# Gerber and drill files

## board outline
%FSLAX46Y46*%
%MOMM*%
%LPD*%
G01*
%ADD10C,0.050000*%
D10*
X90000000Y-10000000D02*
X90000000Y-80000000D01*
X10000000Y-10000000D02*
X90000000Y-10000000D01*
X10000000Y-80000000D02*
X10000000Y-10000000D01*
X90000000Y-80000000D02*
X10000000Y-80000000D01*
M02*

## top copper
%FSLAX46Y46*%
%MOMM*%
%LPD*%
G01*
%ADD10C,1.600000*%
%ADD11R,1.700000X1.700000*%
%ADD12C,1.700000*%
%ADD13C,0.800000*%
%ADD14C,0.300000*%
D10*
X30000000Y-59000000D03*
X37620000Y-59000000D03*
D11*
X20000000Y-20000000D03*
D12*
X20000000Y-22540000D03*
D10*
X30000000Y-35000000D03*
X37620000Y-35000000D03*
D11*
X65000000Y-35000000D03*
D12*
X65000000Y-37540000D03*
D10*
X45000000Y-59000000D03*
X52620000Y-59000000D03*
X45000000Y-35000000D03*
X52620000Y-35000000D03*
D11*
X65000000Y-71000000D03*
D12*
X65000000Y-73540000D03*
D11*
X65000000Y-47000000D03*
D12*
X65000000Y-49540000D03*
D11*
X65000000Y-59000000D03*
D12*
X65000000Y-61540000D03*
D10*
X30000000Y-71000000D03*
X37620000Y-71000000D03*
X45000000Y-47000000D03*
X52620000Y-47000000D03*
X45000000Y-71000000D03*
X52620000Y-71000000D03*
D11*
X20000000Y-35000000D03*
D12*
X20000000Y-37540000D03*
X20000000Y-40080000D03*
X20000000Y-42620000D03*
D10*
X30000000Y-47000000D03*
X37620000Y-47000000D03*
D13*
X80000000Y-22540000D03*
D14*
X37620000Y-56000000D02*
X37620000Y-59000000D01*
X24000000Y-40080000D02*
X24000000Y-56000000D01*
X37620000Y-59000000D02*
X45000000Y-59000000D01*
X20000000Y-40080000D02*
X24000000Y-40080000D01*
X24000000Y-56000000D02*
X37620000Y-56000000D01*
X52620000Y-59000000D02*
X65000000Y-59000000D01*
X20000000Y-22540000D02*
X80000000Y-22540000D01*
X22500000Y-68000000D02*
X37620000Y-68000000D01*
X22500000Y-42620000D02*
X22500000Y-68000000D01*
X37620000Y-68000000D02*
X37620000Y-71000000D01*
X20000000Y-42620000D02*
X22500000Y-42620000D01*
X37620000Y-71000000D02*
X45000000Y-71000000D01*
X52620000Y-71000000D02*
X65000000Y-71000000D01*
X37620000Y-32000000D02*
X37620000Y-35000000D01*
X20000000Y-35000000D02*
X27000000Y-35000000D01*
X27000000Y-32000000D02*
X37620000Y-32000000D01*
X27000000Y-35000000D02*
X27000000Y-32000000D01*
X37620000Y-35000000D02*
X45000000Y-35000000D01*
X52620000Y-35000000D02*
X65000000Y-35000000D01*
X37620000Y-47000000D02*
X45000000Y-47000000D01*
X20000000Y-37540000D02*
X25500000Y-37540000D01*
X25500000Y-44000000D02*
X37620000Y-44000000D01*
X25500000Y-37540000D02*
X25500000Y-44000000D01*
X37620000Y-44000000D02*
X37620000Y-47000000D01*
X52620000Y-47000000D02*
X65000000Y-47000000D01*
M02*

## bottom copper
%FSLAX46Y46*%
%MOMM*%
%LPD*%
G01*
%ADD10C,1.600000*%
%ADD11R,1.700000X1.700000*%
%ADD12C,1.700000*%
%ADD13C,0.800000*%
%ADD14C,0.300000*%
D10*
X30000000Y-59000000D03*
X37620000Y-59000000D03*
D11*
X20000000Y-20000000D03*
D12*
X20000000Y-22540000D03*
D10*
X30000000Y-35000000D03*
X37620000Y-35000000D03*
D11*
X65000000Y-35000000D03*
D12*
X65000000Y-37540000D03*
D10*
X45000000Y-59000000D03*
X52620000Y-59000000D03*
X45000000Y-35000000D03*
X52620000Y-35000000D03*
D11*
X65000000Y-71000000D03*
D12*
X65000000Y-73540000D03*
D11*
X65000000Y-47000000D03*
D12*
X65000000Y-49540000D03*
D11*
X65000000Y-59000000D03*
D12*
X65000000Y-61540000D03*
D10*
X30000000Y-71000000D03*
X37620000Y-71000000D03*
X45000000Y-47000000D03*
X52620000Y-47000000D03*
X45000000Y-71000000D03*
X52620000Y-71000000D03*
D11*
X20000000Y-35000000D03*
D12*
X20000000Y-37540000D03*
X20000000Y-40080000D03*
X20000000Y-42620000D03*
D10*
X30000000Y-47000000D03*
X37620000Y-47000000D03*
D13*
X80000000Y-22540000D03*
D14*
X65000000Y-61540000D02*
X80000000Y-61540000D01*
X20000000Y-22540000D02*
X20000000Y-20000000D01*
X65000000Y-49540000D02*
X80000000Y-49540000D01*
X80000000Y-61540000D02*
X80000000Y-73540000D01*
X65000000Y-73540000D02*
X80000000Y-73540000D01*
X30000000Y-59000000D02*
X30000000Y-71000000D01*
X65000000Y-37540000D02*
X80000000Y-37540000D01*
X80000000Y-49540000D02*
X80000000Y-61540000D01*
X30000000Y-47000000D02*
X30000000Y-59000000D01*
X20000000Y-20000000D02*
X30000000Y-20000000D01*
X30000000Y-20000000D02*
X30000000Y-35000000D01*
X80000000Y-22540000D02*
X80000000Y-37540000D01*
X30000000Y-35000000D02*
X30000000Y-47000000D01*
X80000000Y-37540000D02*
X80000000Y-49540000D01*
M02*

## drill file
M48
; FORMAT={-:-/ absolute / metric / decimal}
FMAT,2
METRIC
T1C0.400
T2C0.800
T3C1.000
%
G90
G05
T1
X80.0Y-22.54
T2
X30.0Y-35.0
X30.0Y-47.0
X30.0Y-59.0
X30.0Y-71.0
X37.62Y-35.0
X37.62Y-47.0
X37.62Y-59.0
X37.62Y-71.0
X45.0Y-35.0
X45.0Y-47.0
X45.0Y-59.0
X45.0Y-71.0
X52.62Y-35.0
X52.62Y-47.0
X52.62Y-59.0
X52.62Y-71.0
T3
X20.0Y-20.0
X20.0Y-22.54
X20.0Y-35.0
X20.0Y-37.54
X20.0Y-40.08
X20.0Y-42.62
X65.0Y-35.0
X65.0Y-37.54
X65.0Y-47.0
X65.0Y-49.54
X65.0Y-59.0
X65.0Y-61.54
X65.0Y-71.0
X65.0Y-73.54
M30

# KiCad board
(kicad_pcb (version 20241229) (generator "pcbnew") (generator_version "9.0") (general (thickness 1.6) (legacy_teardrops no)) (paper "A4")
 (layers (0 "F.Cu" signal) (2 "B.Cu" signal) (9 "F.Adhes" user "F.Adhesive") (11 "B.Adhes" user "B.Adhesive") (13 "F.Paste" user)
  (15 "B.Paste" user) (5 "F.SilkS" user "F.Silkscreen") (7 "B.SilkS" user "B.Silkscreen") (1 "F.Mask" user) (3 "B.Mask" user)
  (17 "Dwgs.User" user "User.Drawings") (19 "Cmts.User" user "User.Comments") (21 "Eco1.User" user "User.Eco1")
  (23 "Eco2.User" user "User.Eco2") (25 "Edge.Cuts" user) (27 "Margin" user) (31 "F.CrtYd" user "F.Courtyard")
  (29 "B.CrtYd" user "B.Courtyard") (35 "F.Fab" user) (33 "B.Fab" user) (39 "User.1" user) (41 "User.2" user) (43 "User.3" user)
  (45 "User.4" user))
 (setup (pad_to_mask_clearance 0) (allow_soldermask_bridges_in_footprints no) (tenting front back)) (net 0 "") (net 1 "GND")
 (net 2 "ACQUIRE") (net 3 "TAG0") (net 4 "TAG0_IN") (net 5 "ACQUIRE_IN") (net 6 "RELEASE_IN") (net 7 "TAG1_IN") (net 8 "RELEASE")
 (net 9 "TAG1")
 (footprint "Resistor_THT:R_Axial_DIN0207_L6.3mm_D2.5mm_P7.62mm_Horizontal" (layer "F.Cu") (at 30 59)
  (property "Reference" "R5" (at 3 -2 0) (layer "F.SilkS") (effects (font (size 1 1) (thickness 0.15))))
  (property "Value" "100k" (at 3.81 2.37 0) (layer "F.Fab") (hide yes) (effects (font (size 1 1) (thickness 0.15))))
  (pad "1" thru_hole circle (at 0 0) (size 1.6 1.6) (drill 0.8) (layers "*.Cu" "*.Mask") (remove_unused_layers no) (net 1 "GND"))
  (pad "2" thru_hole circle (at 7.62 0) (size 1.6 1.6) (drill 0.8) (layers "*.Cu" "*.Mask") (remove_unused_layers no) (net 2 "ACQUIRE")))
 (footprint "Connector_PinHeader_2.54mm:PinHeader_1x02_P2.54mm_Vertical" (layer "F.Cu") (at 20 20)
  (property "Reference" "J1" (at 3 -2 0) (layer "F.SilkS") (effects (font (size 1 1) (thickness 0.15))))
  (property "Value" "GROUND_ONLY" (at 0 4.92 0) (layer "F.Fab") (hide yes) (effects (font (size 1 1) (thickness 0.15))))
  (pad "1" thru_hole rect (at 0 0) (size 1.7 1.7) (drill 1) (layers "*.Cu" "*.Mask") (remove_unused_layers no) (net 1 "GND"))
  (pad "2" thru_hole circle (at 0 2.54) (size 1.7 1.7) (drill 1) (layers "*.Cu" "*.Mask") (remove_unused_layers no) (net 1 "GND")))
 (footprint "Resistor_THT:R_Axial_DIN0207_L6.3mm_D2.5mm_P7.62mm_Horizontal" (layer "F.Cu") (at 30 35)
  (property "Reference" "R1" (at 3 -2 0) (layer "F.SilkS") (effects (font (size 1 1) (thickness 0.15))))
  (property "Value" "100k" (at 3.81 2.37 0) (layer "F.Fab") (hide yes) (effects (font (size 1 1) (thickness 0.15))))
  (pad "1" thru_hole circle (at 0 0) (size 1.6 1.6) (drill 0.8) (layers "*.Cu" "*.Mask") (remove_unused_layers no) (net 1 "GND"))
  (pad "2" thru_hole circle (at 7.62 0) (size 1.6 1.6) (drill 0.8) (layers "*.Cu" "*.Mask") (remove_unused_layers no) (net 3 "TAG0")))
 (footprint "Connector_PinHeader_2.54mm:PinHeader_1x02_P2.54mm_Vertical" (layer "F.Cu") (at 65 35)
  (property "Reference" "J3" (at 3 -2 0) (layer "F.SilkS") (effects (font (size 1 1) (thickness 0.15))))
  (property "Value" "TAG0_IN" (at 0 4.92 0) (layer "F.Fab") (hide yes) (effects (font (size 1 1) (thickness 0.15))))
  (pad "1" thru_hole rect (at 0 0) (size 1.7 1.7) (drill 1) (layers "*.Cu" "*.Mask") (remove_unused_layers no) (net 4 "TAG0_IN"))
  (pad "2" thru_hole circle (at 0 2.54) (size 1.7 1.7) (drill 1) (layers "*.Cu" "*.Mask") (remove_unused_layers no) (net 1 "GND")))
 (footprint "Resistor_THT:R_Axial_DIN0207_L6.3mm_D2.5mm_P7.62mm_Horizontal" (layer "F.Cu") (at 45 59)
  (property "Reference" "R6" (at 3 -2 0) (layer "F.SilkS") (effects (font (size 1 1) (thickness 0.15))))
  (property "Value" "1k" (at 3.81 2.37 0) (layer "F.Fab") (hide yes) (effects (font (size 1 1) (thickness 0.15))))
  (pad "1" thru_hole circle (at 0 0) (size 1.6 1.6) (drill 0.8) (layers "*.Cu" "*.Mask") (remove_unused_layers no) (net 2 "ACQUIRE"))
  (pad "2" thru_hole circle (at 7.62 0) (size 1.6 1.6) (drill 0.8) (layers "*.Cu" "*.Mask") (remove_unused_layers no) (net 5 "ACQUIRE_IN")))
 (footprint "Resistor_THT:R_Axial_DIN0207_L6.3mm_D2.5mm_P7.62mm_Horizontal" (layer "F.Cu") (at 45 35)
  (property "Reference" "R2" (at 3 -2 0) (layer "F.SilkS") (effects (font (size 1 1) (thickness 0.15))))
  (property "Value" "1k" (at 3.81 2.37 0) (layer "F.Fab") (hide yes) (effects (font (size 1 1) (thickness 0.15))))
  (pad "1" thru_hole circle (at 0 0) (size 1.6 1.6) (drill 0.8) (layers "*.Cu" "*.Mask") (remove_unused_layers no) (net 3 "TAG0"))
  (pad "2" thru_hole circle (at 7.62 0) (size 1.6 1.6) (drill 0.8) (layers "*.Cu" "*.Mask") (remove_unused_layers no) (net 4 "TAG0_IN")))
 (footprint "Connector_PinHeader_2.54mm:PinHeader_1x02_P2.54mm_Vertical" (layer "F.Cu") (at 65 71)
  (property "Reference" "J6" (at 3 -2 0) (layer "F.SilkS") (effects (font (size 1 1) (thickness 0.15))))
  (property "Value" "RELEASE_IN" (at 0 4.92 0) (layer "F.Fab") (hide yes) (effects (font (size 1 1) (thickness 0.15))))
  (pad "1" thru_hole rect (at 0 0) (size 1.7 1.7) (drill 1) (layers "*.Cu" "*.Mask") (remove_unused_layers no) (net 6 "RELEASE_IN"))
  (pad "2" thru_hole circle (at 0 2.54) (size 1.7 1.7) (drill 1) (layers "*.Cu" "*.Mask") (remove_unused_layers no) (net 1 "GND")))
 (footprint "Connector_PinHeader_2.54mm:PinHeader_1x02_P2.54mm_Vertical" (layer "F.Cu") (at 65 47)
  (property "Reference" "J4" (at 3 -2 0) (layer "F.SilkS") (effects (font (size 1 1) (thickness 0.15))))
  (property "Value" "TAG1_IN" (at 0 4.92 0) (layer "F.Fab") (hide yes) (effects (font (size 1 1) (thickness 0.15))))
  (pad "1" thru_hole rect (at 0 0) (size 1.7 1.7) (drill 1) (layers "*.Cu" "*.Mask") (remove_unused_layers no) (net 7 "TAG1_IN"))
  (pad "2" thru_hole circle (at 0 2.54) (size 1.7 1.7) (drill 1) (layers "*.Cu" "*.Mask") (remove_unused_layers no) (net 1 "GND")))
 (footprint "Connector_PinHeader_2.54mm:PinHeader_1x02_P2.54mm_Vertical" (layer "F.Cu") (at 65 59)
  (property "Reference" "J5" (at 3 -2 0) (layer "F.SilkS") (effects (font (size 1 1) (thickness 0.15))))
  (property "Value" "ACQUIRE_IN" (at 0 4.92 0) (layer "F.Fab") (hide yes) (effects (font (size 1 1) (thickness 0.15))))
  (pad "1" thru_hole rect (at 0 0) (size 1.7 1.7) (drill 1) (layers "*.Cu" "*.Mask") (remove_unused_layers no) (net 5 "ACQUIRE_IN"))
  (pad "2" thru_hole circle (at 0 2.54) (size 1.7 1.7) (drill 1) (layers "*.Cu" "*.Mask") (remove_unused_layers no) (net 1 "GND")))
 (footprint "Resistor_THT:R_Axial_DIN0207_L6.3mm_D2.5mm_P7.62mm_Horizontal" (layer "F.Cu") (at 30 71)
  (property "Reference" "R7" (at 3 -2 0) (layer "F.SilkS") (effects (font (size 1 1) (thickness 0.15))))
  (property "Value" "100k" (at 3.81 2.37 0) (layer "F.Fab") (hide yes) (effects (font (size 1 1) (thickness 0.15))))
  (pad "1" thru_hole circle (at 0 0) (size 1.6 1.6) (drill 0.8) (layers "*.Cu" "*.Mask") (remove_unused_layers no) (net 1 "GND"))
  (pad "2" thru_hole circle (at 7.62 0) (size 1.6 1.6) (drill 0.8) (layers "*.Cu" "*.Mask") (remove_unused_layers no) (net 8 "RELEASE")))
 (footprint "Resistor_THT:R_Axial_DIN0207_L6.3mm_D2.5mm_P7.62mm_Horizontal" (layer "F.Cu") (at 45 47)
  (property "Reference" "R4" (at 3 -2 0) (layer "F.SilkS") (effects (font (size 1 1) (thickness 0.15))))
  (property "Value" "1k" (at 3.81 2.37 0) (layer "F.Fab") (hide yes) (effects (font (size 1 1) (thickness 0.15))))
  (pad "1" thru_hole circle (at 0 0) (size 1.6 1.6) (drill 0.8) (layers "*.Cu" "*.Mask") (remove_unused_layers no) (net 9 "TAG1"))
  (pad "2" thru_hole circle (at 7.62 0) (size 1.6 1.6) (drill 0.8) (layers "*.Cu" "*.Mask") (remove_unused_layers no) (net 7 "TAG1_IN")))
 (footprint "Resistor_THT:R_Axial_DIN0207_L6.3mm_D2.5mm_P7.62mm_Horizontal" (layer "F.Cu") (at 45 71)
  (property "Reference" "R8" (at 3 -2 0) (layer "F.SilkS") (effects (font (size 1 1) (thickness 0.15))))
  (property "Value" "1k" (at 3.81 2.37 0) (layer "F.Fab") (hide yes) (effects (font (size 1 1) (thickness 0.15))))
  (pad "1" thru_hole circle (at 0 0) (size 1.6 1.6) (drill 0.8) (layers "*.Cu" "*.Mask") (remove_unused_layers no) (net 8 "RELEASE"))
  (pad "2" thru_hole circle (at 7.62 0) (size 1.6 1.6) (drill 0.8) (layers "*.Cu" "*.Mask") (remove_unused_layers no) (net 6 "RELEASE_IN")))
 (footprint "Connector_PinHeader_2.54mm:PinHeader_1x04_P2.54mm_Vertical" (layer "F.Cu") (at 20 35)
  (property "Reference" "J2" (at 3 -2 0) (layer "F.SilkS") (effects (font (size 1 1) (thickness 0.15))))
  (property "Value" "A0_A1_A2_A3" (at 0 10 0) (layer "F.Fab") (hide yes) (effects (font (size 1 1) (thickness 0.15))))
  (pad "1" thru_hole rect (at 0 0) (size 1.7 1.7) (drill 1) (layers "*.Cu" "*.Mask") (remove_unused_layers no) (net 3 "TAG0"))
  (pad "2" thru_hole circle (at 0 2.54) (size 1.7 1.7) (drill 1) (layers "*.Cu" "*.Mask") (remove_unused_layers no) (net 9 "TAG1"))
  (pad "3" thru_hole circle (at 0 5.08) (size 1.7 1.7) (drill 1) (layers "*.Cu" "*.Mask") (remove_unused_layers no) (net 2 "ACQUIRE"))
  (pad "4" thru_hole circle (at 0 7.62) (size 1.7 1.7) (drill 1) (layers "*.Cu" "*.Mask") (remove_unused_layers no) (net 8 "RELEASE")))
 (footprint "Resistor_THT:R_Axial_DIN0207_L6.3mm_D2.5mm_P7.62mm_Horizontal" (layer "F.Cu") (at 30 47)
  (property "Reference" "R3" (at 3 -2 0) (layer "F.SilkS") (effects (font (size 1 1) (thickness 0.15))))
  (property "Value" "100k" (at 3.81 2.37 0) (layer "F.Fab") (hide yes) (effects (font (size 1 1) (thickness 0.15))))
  (pad "1" thru_hole circle (at 0 0) (size 1.6 1.6) (drill 0.8) (layers "*.Cu" "*.Mask") (remove_unused_layers no) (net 1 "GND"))
  (pad "2" thru_hole circle (at 7.62 0) (size 1.6 1.6) (drill 0.8) (layers "*.Cu" "*.Mask") (remove_unused_layers no) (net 9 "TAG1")))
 (gr_line (start 90 10) (end 90 80) (stroke (width 0.05) (type default)) (layer "Edge.Cuts"))
 (gr_line (start 10 10) (end 90 10) (stroke (width 0.05) (type default)) (layer "Edge.Cuts"))
 (gr_line (start 10 80) (end 10 10) (stroke (width 0.05) (type default)) (layer "Edge.Cuts"))
 (gr_line (start 90 80) (end 10 80) (stroke (width 0.05) (type default)) (layer "Edge.Cuts"))
 (segment (start 37.62 56) (end 37.62 59) (width 0.3) (layer "F.Cu") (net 2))
 (segment (start 24 40.08) (end 24 56) (width 0.3) (layer "F.Cu") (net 2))
 (segment (start 37.62 59) (end 45 59) (width 0.3) (layer "F.Cu") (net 2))
 (segment (start 20 40.08) (end 24 40.08) (width 0.3) (layer "F.Cu") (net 2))
 (segment (start 24 56) (end 37.62 56) (width 0.3) (layer "F.Cu") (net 2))
 (segment (start 52.62 59) (end 65 59) (width 0.3) (layer "F.Cu") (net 5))
 (segment (start 20 22.54) (end 80 22.54) (width 0.3) (layer "F.Cu") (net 1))
 (via (at 80 22.54) (size 0.8) (drill 0.4) (layers "F.Cu" "B.Cu") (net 1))
 (segment (start 65 61.54) (end 80 61.54) (width 0.3) (layer "B.Cu") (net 1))
 (segment (start 20 22.54) (end 20 20) (width 0.3) (layer "B.Cu") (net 1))
 (segment (start 65 49.54) (end 80 49.54) (width 0.3) (layer "B.Cu") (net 1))
 (segment (start 80 61.54) (end 80 73.54) (width 0.3) (layer "B.Cu") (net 1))
 (segment (start 65 73.54) (end 80 73.54) (width 0.3) (layer "B.Cu") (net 1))
 (segment (start 30 59) (end 30 71) (width 0.3) (layer "B.Cu") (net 1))
 (segment (start 65 37.54) (end 80 37.54) (width 0.3) (layer "B.Cu") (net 1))
 (segment (start 80 49.54) (end 80 61.54) (width 0.3) (layer "B.Cu") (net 1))
 (segment (start 30 47) (end 30 59) (width 0.3) (layer "B.Cu") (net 1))
 (segment (start 20 20) (end 30 20) (width 0.3) (layer "B.Cu") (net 1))
 (segment (start 30 20) (end 30 35) (width 0.3) (layer "B.Cu") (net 1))
 (segment (start 80 22.54) (end 80 37.54) (width 0.3) (layer "B.Cu") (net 1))
 (segment (start 30 35) (end 30 47) (width 0.3) (layer "B.Cu") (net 1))
 (segment (start 80 37.54) (end 80 49.54) (width 0.3) (layer "B.Cu") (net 1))
 (segment (start 22.5 68) (end 37.62 68) (width 0.3) (layer "F.Cu") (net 8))
 (segment (start 22.5 42.62) (end 22.5 68) (width 0.3) (layer "F.Cu") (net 8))
 (segment (start 37.62 68) (end 37.62 71) (width 0.3) (layer "F.Cu") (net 8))
 (segment (start 20 42.62) (end 22.5 42.62) (width 0.3) (layer "F.Cu") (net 8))
 (segment (start 37.62 71) (end 45 71) (width 0.3) (layer "F.Cu") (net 8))
 (segment (start 52.62 71) (end 65 71) (width 0.3) (layer "F.Cu") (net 6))
 (segment (start 37.62 32) (end 37.62 35) (width 0.3) (layer "F.Cu") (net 3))
 (segment (start 20 35) (end 27 35) (width 0.3) (layer "F.Cu") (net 3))
 (segment (start 27 32) (end 37.62 32) (width 0.3) (layer "F.Cu") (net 3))
 (segment (start 27 35) (end 27 32) (width 0.3) (layer "F.Cu") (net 3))
 (segment (start 37.62 35) (end 45 35) (width 0.3) (layer "F.Cu") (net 3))
 (segment (start 52.62 35) (end 65 35) (width 0.3) (layer "F.Cu") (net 4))
 (segment (start 37.62 47) (end 45 47) (width 0.3) (layer "F.Cu") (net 9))
 (segment (start 20 37.54) (end 25.5 37.54) (width 0.3) (layer "F.Cu") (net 9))
 (segment (start 25.5 44) (end 37.62 44) (width 0.3) (layer "F.Cu") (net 9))
 (segment (start 25.5 37.54) (end 25.5 44) (width 0.3) (layer "F.Cu") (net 9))
 (segment (start 37.62 44) (end 37.62 47) (width 0.3) (layer "F.Cu") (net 9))
 (segment (start 52.62 47) (end 65 47) (width 0.3) (layer "F.Cu") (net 7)))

